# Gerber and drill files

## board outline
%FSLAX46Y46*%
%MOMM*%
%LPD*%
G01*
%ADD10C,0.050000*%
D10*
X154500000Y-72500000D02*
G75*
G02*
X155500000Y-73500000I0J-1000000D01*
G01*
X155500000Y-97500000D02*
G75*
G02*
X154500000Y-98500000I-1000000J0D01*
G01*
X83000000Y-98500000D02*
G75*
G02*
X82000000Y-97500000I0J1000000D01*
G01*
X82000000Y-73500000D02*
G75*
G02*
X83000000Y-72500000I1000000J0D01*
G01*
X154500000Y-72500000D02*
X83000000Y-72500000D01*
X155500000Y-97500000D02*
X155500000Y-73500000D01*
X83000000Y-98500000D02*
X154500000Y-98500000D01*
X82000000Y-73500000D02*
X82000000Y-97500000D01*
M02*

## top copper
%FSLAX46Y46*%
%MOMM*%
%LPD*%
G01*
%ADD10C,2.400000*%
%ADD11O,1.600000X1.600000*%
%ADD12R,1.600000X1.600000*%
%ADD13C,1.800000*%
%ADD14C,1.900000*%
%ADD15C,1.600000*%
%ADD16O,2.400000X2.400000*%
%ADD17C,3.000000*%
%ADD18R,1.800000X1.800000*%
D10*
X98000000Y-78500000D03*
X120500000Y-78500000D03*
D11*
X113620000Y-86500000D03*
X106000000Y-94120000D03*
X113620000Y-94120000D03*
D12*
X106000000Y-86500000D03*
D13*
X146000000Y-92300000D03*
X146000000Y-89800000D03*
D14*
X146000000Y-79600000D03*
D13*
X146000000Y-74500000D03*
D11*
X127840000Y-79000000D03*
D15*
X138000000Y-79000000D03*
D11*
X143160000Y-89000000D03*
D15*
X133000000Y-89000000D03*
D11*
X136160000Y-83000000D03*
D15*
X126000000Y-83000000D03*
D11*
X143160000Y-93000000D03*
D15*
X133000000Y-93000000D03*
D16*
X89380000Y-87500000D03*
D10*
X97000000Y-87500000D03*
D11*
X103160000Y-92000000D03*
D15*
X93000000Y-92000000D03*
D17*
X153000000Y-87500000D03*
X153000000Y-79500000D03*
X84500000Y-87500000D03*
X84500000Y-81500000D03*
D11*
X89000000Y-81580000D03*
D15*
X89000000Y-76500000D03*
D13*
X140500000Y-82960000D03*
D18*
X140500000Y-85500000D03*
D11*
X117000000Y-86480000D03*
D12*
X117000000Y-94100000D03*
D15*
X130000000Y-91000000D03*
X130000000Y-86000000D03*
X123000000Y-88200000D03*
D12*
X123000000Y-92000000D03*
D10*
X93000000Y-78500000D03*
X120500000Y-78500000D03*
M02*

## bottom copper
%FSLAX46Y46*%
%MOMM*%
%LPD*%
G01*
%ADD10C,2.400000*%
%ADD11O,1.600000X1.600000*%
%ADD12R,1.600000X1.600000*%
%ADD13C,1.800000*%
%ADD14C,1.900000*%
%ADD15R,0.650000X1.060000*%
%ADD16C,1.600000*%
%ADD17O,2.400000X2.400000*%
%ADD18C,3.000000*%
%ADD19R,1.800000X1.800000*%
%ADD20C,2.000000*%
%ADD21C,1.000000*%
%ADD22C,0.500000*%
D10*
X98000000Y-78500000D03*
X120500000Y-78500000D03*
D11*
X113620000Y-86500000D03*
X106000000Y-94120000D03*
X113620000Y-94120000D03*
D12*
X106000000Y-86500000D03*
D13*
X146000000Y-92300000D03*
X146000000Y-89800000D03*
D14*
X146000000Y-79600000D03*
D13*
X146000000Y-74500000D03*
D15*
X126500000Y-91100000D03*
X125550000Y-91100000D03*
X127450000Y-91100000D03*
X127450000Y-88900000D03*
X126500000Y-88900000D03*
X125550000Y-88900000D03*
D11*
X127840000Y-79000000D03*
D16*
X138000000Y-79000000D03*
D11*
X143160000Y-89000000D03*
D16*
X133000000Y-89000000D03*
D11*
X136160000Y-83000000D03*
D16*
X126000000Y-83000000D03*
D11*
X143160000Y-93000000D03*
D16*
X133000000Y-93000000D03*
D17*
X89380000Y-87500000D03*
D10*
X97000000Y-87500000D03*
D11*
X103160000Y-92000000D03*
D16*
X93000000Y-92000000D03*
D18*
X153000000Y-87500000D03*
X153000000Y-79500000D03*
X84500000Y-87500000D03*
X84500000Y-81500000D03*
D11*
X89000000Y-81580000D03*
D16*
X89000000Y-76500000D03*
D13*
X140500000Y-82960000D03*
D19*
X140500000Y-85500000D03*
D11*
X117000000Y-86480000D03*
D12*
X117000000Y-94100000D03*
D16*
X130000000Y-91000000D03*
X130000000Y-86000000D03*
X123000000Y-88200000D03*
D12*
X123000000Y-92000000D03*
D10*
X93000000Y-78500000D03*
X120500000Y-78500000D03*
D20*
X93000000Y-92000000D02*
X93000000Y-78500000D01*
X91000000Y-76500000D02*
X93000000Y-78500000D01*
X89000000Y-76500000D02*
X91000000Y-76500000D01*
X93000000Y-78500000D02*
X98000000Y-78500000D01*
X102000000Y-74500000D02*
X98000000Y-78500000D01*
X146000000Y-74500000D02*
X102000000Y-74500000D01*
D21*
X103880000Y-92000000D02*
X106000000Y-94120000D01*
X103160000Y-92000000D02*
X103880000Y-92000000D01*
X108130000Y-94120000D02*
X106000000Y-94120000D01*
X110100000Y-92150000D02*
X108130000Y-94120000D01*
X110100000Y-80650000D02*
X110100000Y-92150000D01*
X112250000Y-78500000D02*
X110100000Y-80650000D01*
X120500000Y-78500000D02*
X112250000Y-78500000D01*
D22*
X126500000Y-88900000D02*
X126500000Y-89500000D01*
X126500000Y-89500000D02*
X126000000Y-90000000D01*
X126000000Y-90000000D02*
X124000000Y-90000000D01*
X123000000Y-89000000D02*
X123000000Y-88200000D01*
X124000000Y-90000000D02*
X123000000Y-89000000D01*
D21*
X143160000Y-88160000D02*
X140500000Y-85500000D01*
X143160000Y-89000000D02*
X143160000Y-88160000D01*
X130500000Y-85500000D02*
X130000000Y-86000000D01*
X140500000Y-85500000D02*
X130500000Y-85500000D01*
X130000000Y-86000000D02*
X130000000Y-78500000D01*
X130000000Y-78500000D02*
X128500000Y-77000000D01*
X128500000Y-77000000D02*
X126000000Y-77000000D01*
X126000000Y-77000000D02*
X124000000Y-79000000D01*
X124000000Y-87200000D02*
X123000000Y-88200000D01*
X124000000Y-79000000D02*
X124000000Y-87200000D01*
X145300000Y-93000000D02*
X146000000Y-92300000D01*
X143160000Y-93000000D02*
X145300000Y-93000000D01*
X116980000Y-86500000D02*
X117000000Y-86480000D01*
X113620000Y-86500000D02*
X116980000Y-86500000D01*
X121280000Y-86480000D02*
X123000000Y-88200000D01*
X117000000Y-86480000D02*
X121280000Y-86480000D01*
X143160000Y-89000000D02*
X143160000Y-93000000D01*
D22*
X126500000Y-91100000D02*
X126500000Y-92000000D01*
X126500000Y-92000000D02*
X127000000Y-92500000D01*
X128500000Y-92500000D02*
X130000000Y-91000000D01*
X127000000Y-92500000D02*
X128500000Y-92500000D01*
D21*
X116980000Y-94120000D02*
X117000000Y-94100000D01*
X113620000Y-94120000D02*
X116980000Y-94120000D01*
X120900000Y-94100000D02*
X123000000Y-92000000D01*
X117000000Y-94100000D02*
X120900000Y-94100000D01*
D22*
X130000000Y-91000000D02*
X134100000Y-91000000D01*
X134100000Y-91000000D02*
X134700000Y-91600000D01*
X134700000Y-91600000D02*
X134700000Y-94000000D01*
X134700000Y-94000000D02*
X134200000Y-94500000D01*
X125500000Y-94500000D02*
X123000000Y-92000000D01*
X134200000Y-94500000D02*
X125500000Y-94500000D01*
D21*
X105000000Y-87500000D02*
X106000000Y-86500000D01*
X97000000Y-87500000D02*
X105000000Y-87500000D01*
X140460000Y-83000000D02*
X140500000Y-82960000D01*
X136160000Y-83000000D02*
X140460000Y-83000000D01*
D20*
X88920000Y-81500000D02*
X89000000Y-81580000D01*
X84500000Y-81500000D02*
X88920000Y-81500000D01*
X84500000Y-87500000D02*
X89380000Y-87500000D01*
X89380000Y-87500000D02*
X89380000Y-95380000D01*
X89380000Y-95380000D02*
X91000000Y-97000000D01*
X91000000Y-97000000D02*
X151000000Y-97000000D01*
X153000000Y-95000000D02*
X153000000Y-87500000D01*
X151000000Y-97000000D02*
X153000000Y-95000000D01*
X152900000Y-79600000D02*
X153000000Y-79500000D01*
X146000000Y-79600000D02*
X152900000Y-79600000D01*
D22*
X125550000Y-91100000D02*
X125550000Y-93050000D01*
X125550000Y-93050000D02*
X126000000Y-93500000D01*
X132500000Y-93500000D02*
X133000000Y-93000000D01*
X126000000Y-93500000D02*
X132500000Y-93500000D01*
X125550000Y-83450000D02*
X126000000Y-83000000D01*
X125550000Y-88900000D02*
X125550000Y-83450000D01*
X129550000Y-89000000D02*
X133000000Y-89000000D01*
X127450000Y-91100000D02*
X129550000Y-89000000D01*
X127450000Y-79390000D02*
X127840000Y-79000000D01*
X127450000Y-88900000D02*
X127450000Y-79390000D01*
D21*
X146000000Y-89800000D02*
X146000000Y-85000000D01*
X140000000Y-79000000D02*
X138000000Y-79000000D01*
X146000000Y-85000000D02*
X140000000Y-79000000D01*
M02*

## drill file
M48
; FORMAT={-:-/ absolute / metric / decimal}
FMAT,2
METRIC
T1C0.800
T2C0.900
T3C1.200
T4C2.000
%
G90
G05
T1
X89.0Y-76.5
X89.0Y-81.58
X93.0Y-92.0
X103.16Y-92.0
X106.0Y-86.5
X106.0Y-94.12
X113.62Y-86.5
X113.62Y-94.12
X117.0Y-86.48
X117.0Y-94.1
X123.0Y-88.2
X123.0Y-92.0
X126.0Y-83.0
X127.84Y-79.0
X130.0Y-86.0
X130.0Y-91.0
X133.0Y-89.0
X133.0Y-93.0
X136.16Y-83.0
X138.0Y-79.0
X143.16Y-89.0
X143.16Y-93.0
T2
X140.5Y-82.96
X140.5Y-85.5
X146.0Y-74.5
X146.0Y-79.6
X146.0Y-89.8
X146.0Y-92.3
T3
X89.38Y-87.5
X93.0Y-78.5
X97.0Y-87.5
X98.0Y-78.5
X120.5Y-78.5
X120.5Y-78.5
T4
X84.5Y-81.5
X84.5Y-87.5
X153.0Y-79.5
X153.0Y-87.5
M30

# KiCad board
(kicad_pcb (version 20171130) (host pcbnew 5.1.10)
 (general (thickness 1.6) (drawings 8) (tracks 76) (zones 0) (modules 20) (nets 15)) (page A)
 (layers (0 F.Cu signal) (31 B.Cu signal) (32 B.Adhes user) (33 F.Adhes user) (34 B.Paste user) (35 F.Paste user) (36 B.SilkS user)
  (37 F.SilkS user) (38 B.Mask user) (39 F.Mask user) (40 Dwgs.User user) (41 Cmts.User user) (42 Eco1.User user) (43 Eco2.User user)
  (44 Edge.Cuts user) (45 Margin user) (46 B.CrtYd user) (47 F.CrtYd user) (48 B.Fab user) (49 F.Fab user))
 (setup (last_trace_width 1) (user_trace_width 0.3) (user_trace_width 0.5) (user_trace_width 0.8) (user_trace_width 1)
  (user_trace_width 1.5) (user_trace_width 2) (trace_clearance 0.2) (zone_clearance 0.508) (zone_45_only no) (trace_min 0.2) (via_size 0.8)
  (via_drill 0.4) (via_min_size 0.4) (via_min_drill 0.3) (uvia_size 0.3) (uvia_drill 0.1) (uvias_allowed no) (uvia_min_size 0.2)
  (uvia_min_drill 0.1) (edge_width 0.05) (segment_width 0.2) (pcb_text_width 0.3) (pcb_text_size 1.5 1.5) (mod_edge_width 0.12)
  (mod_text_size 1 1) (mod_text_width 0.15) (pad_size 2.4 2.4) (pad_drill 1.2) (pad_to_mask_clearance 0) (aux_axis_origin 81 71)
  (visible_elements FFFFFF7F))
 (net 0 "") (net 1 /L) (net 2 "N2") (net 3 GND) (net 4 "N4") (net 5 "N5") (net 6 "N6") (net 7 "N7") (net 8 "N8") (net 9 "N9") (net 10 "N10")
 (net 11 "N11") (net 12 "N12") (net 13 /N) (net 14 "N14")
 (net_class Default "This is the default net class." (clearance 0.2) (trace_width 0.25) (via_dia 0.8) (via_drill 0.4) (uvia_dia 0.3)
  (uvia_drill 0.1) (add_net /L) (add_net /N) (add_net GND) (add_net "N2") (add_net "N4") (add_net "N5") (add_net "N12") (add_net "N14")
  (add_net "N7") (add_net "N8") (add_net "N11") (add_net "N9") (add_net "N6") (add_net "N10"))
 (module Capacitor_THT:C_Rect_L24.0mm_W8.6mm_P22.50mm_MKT (layer F.Cu) (at 120.5 78.5 180)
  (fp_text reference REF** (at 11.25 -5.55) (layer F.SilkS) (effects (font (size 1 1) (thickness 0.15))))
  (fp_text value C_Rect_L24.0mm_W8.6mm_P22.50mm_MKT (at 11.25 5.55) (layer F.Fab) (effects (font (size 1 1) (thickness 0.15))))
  (pad 2 thru_hole circle (at 22.5 0 180) (size 2.4 2.4) (drill 1.2) (layers *.Cu *.Mask) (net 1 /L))
  (pad 1 thru_hole circle (at 0 0 180) (size 2.4 2.4) (drill 1.2) (layers *.Cu *.Mask) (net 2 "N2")))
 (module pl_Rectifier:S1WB (layer F.Cu) (at 106 86.5)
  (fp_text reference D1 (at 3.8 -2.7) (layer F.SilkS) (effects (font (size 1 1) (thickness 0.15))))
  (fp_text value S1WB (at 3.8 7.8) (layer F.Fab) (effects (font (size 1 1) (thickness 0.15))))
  (pad 4 thru_hole oval (at 7.62 0) (size 1.6 1.6) (drill 0.8) (layers *.Cu *.Mask) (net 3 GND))
  (pad 2 thru_hole oval (at 0 7.62) (size 1.6 1.6) (drill 0.8) (layers *.Cu *.Mask) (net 2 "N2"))
  (pad 3 thru_hole oval (at 7.62 7.62) (size 1.6 1.6) (drill 0.8) (layers *.Cu *.Mask) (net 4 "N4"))
  (pad 1 thru_hole rect (at 0 0) (size 1.6 1.6) (drill 0.8) (layers *.Cu *.Mask) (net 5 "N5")))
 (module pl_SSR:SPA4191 (layer F.Cu) (at 146 74.5 270)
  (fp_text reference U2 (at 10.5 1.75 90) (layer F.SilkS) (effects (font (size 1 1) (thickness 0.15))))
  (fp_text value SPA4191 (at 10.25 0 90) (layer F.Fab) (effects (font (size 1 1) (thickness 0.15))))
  (pad 4 thru_hole circle (at 17.8 0 270) (size 1.8 1.8) (drill 0.9) (layers *.Cu *.Mask) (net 3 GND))
  (pad 3 thru_hole circle (at 15.3 0 270) (size 1.8 1.8) (drill 0.9) (layers *.Cu *.Mask) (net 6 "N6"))
  (pad 2 thru_hole circle (at 5.1 0 270) (size 1.9 1.9) (drill 0.9) (layers *.Cu *.Mask) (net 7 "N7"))
  (pad 1 thru_hole circle (at 0 0 270) (size 1.8 1.8) (drill 0.9) (layers *.Cu *.Mask) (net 1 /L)))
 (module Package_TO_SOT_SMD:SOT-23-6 (layer B.Cu) (at 126.5 90 270)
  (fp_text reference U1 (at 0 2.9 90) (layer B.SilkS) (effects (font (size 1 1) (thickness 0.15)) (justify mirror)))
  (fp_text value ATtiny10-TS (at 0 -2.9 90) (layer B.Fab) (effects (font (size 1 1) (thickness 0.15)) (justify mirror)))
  (pad 5 smd rect (at 1.1 0 270) (size 1.06 0.65) (layers B.Cu B.Paste B.Mask) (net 4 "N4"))
  (pad 6 smd rect (at 1.1 0.95 270) (size 1.06 0.65) (layers B.Cu B.Paste B.Mask) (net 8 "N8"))
  (pad 4 smd rect (at 1.1 -0.95 270) (size 1.06 0.65) (layers B.Cu B.Paste B.Mask) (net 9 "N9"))
  (pad 3 smd rect (at -1.1 -0.95 270) (size 1.06 0.65) (layers B.Cu B.Paste B.Mask) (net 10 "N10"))
  (pad 2 smd rect (at -1.1 0 270) (size 1.06 0.65) (layers B.Cu B.Paste B.Mask) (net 3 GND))
  (pad 1 smd rect (at -1.1 0.95 270) (size 1.06 0.65) (layers B.Cu B.Paste B.Mask) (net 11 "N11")))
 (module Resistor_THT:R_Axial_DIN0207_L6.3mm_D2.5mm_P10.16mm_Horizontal (layer F.Cu) (at 138 79 180)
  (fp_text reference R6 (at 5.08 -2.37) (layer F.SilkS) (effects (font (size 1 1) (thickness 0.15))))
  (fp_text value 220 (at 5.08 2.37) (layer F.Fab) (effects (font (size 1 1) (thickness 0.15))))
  (pad 2 thru_hole oval (at 10.16 0 180) (size 1.6 1.6) (drill 0.8) (layers *.Cu *.Mask) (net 10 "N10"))
  (pad 1 thru_hole circle (at 0 0 180) (size 1.6 1.6) (drill 0.8) (layers *.Cu *.Mask) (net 6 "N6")))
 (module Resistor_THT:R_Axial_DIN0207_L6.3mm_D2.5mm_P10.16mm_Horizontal (layer F.Cu) (at 133 89)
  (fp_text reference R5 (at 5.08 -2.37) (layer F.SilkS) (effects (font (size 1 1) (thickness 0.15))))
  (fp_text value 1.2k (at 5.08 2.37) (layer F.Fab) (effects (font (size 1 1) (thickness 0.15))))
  (pad 2 thru_hole oval (at 10.16 0) (size 1.6 1.6) (drill 0.8) (layers *.Cu *.Mask) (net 3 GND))
  (pad 1 thru_hole circle (at 0 0) (size 1.6 1.6) (drill 0.8) (layers *.Cu *.Mask) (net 9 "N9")))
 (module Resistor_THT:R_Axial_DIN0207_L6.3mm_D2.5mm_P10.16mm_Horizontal (layer F.Cu) (at 126 83)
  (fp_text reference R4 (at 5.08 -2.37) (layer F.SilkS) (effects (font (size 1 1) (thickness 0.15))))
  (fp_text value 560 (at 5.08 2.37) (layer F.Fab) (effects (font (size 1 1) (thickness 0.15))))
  (pad 2 thru_hole oval (at 10.16 0) (size 1.6 1.6) (drill 0.8) (layers *.Cu *.Mask) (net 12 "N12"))
  (pad 1 thru_hole circle (at 0 0) (size 1.6 1.6) (drill 0.8) (layers *.Cu *.Mask) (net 11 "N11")))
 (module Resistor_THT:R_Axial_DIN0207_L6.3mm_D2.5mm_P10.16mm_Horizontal (layer F.Cu) (at 133 93)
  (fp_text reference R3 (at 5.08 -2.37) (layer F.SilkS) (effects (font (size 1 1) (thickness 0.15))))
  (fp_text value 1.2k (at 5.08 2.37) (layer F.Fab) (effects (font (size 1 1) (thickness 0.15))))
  (pad 2 thru_hole oval (at 10.16 0) (size 1.6 1.6) (drill 0.8) (layers *.Cu *.Mask) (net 3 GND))
  (pad 1 thru_hole circle (at 0 0) (size 1.6 1.6) (drill 0.8) (layers *.Cu *.Mask) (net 8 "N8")))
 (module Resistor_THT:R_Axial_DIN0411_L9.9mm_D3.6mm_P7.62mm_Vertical (layer F.Cu) (at 97 87.5 180)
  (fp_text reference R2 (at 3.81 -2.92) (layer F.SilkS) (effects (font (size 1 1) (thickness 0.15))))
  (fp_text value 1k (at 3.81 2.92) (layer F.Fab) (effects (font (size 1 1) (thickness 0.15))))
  (pad 2 thru_hole oval (at 7.62 0 180) (size 2.4 2.4) (drill 1.2) (layers *.Cu *.Mask) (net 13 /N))
  (pad 1 thru_hole circle (at 0 0 180) (size 2.4 2.4) (drill 1.2) (layers *.Cu *.Mask) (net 5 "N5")))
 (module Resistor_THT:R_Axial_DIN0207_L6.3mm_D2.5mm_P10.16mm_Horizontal (layer F.Cu) (at 93 92)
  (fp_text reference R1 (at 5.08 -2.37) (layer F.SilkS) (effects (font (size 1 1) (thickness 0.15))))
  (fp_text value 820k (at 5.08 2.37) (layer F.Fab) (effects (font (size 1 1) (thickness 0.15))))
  (pad 2 thru_hole oval (at 10.16 0) (size 1.6 1.6) (drill 0.8) (layers *.Cu *.Mask) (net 2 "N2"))
  (pad 1 thru_hole circle (at 0 0) (size 1.6 1.6) (drill 0.8) (layers *.Cu *.Mask) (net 1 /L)))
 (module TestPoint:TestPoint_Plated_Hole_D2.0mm (layer F.Cu) (at 153 87.5)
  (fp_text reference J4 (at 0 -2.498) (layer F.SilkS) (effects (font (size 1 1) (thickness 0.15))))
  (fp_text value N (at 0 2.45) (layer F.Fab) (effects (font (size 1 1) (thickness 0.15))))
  (pad 1 thru_hole circle (at 0 0) (size 3 3) (drill 2) (layers *.Cu *.Mask) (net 13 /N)))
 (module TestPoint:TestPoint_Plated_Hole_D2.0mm (layer F.Cu) (at 153 79.5)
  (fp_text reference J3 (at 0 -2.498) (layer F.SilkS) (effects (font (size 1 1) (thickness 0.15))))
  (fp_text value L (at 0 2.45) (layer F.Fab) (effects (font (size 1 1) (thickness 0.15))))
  (pad 1 thru_hole circle (at 0 0) (size 3 3) (drill 2) (layers *.Cu *.Mask) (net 7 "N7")))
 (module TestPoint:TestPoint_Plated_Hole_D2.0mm (layer F.Cu) (at 84.5 87.5)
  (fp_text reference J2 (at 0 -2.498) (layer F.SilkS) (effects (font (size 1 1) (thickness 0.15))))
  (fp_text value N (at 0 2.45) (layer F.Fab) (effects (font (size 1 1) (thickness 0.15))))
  (pad 1 thru_hole circle (at 0 0) (size 3 3) (drill 2) (layers *.Cu *.Mask) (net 13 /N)))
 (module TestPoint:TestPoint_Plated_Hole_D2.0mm (layer F.Cu) (at 84.5 81.5)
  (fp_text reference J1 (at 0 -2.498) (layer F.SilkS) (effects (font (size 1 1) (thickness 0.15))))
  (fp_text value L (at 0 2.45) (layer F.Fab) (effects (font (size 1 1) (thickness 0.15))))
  (pad 1 thru_hole circle (at 0 0) (size 3 3) (drill 2) (layers *.Cu *.Mask) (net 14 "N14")))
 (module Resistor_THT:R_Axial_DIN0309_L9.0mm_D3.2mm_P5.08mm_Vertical (layer F.Cu) (at 89 76.5 270)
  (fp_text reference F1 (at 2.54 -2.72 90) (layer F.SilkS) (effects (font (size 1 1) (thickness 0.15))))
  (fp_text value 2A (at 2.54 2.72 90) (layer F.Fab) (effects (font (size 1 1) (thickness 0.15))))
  (pad 2 thru_hole oval (at 5.08 0 270) (size 1.6 1.6) (drill 0.8) (layers *.Cu *.Mask) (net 14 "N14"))
  (pad 1 thru_hole circle (at 0 0 270) (size 1.6 1.6) (drill 0.8) (layers *.Cu *.Mask) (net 1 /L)))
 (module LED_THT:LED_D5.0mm (layer F.Cu) (at 140.5 85.5 90)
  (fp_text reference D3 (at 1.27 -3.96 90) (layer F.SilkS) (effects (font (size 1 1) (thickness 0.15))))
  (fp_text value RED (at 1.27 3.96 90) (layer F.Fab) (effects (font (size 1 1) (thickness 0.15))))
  (pad 2 thru_hole circle (at 2.54 0 90) (size 1.8 1.8) (drill 0.9) (layers *.Cu *.Mask) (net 12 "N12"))
  (pad 1 thru_hole rect (at 0 0 90) (size 1.8 1.8) (drill 0.9) (layers *.Cu *.Mask) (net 3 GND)))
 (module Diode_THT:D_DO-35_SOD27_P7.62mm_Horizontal (layer F.Cu) (at 117 94.1 90)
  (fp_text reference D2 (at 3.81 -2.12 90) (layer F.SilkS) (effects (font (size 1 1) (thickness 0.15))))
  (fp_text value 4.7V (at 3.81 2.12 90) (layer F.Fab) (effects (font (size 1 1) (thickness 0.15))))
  (pad 2 thru_hole oval (at 7.62 0 90) (size 1.6 1.6) (drill 0.8) (layers *.Cu *.Mask) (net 3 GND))
  (pad 1 thru_hole rect (at 0 0 90) (size 1.6 1.6) (drill 0.8) (layers *.Cu *.Mask) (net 4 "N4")))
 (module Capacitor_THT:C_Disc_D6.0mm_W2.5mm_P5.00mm (layer F.Cu) (at 130 86 270)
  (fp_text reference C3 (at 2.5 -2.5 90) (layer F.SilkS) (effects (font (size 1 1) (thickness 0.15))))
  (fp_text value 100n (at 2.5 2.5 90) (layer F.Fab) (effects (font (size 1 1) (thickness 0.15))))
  (pad 2 thru_hole circle (at 5 0 270) (size 1.6 1.6) (drill 0.8) (layers *.Cu *.Mask) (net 4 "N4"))
  (pad 1 thru_hole circle (at 0 0 270) (size 1.6 1.6) (drill 0.8) (layers *.Cu *.Mask) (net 3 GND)))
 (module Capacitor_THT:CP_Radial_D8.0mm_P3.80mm (layer F.Cu) (at 123 92 90)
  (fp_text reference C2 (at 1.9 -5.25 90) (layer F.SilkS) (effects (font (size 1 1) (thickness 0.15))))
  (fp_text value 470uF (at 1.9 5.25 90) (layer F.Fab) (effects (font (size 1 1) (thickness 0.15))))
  (pad 2 thru_hole circle (at 3.8 0 90) (size 1.6 1.6) (drill 0.8) (layers *.Cu *.Mask) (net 3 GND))
  (pad 1 thru_hole rect (at 0 0 90) (size 1.6 1.6) (drill 0.8) (layers *.Cu *.Mask) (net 4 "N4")))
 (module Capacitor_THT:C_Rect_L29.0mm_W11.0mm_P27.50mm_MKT (layer F.Cu) (at 120.5 78.5 180)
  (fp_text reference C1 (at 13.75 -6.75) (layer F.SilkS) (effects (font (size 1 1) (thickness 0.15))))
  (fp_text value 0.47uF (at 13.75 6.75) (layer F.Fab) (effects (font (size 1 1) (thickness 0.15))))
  (pad 2 thru_hole circle (at 27.5 0 180) (size 2.4 2.4) (drill 1.2) (layers *.Cu *.Mask) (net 1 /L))
  (pad 1 thru_hole circle (at 0 0 180) (size 2.4 2.4) (drill 1.2) (layers *.Cu *.Mask) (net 2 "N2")))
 (gr_arc (start 154.5 73.5) (end 155.5 73.5) (angle -90) (layer Edge.Cuts) (width 0.05))
 (gr_arc (start 154.5 97.5) (end 154.5 98.5) (angle -90) (layer Edge.Cuts) (width 0.05))
 (gr_arc (start 83 97.5) (end 82 97.5) (angle -90) (layer Edge.Cuts) (width 0.05))
 (gr_arc (start 83 73.5) (end 83 72.5) (angle -90) (layer Edge.Cuts) (width 0.05))
 (gr_line (start 154.5 72.5) (end 83 72.5) (layer Edge.Cuts) (width 0.05))
 (gr_line (start 155.5 97.5) (end 155.5 73.5) (layer Edge.Cuts) (width 0.05))
 (gr_line (start 83 98.5) (end 154.5 98.5) (layer Edge.Cuts) (width 0.05))
 (gr_line (start 82 73.5) (end 82 97.5) (layer Edge.Cuts) (width 0.05))
 (segment (start 93 92) (end 93 78.5) (width 2) (layer B.Cu) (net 1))
 (segment (start 91 76.5) (end 93 78.5) (width 2) (layer B.Cu) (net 1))
 (segment (start 89 76.5) (end 91 76.5) (width 2) (layer B.Cu) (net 1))
 (segment (start 93 78.5) (end 98 78.5) (width 2) (layer B.Cu) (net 1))
 (segment (start 102 74.5) (end 98 78.5) (width 2) (layer B.Cu) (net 1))
 (segment (start 146 74.5) (end 102 74.5) (width 2) (layer B.Cu) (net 1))
 (segment (start 103.88 92) (end 106 94.12) (width 1) (layer B.Cu) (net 2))
 (segment (start 103.16 92) (end 103.88 92) (width 1) (layer B.Cu) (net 2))
 (segment (start 108.13 94.12) (end 106 94.12) (width 1) (layer B.Cu) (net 2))
 (segment (start 110.1 92.15) (end 108.13 94.12) (width 1) (layer B.Cu) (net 2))
 (segment (start 110.1 80.65) (end 110.1 92.15) (width 1) (layer B.Cu) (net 2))
 (segment (start 112.25 78.5) (end 110.1 80.65) (width 1) (layer B.Cu) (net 2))
 (segment (start 120.5 78.5) (end 112.25 78.5) (width 1) (layer B.Cu) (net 2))
 (segment (start 126.5 88.9) (end 126.5 89.5) (width 0.5) (layer B.Cu) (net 3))
 (segment (start 126.5 89.5) (end 126 90) (width 0.5) (layer B.Cu) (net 3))
 (segment (start 126 90) (end 124 90) (width 0.5) (layer B.Cu) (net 3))
 (segment (start 123 89) (end 123 88.2) (width 0.5) (layer B.Cu) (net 3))
 (segment (start 124 90) (end 123 89) (width 0.5) (layer B.Cu) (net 3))
 (segment (start 143.16 88.16) (end 140.5 85.5) (width 1) (layer B.Cu) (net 3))
 (segment (start 143.16 89) (end 143.16 88.16) (width 1) (layer B.Cu) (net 3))
 (segment (start 130.5 85.5) (end 130 86) (width 1) (layer B.Cu) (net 3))
 (segment (start 140.5 85.5) (end 130.5 85.5) (width 1) (layer B.Cu) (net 3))
 (segment (start 130 86) (end 130 78.5) (width 1) (layer B.Cu) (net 3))
 (segment (start 130 78.5) (end 128.5 77) (width 1) (layer B.Cu) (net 3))
 (segment (start 128.5 77) (end 126 77) (width 1) (layer B.Cu) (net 3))
 (segment (start 126 77) (end 124 79) (width 1) (layer B.Cu) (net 3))
 (segment (start 124 87.2) (end 123 88.2) (width 1) (layer B.Cu) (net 3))
 (segment (start 124 79) (end 124 87.2) (width 1) (layer B.Cu) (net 3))
 (segment (start 145.3 93) (end 146 92.3) (width 1) (layer B.Cu) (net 3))
 (segment (start 143.16 93) (end 145.3 93) (width 1) (layer B.Cu) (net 3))
 (segment (start 116.98 86.5) (end 117 86.48) (width 1) (layer B.Cu) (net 3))
 (segment (start 113.62 86.5) (end 116.98 86.5) (width 1) (layer B.Cu) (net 3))
 (segment (start 121.28 86.48) (end 123 88.2) (width 1) (layer B.Cu) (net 3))
 (segment (start 117 86.48) (end 121.28 86.48) (width 1) (layer B.Cu) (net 3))
 (segment (start 143.16 89) (end 143.16 93) (width 1) (layer B.Cu) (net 3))
 (segment (start 126.5 91.1) (end 126.5 92) (width 0.5) (layer B.Cu) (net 4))
 (segment (start 126.5 92) (end 127 92.5) (width 0.5) (layer B.Cu) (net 4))
 (segment (start 128.5 92.5) (end 130 91) (width 0.5) (layer B.Cu) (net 4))
 (segment (start 127 92.5) (end 128.5 92.5) (width 0.5) (layer B.Cu) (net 4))
 (segment (start 116.98 94.12) (end 117 94.1) (width 1) (layer B.Cu) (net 4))
 (segment (start 113.62 94.12) (end 116.98 94.12) (width 1) (layer B.Cu) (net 4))
 (segment (start 120.9 94.1) (end 123 92) (width 1) (layer B.Cu) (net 4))
 (segment (start 117 94.1) (end 120.9 94.1) (width 1) (layer B.Cu) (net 4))
 (segment (start 130 91) (end 134.1 91) (width 0.5) (layer B.Cu) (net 4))
 (segment (start 134.1 91) (end 134.7 91.6) (width 0.5) (layer B.Cu) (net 4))
 (segment (start 134.7 91.6) (end 134.7 94) (width 0.5) (layer B.Cu) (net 4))
 (segment (start 134.7 94) (end 134.2 94.5) (width 0.5) (layer B.Cu) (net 4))
 (segment (start 125.5 94.5) (end 123 92) (width 0.5) (layer B.Cu) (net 4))
 (segment (start 134.2 94.5) (end 125.5 94.5) (width 0.5) (layer B.Cu) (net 4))
 (segment (start 105 87.5) (end 106 86.5) (width 1) (layer B.Cu) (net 5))
 (segment (start 97 87.5) (end 105 87.5) (width 1) (layer B.Cu) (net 5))
 (segment (start 140.46 83) (end 140.5 82.96) (width 1) (layer B.Cu) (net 12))
 (segment (start 136.16 83) (end 140.46 83) (width 1) (layer B.Cu) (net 12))
 (segment (start 88.92 81.5) (end 89 81.58) (width 2) (layer B.Cu) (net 14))
 (segment (start 84.5 81.5) (end 88.92 81.5) (width 2) (layer B.Cu) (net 14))
 (segment (start 84.5 87.5) (end 89.38 87.5) (width 2) (layer B.Cu) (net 13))
 (segment (start 89.38 87.5) (end 89.38 95.38) (width 2) (layer B.Cu) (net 13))
 (segment (start 89.38 95.38) (end 91 97) (width 2) (layer B.Cu) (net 13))
 (segment (start 91 97) (end 151 97) (width 2) (layer B.Cu) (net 13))
 (segment (start 153 95) (end 153 87.5) (width 2) (layer B.Cu) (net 13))
 (segment (start 151 97) (end 153 95) (width 2) (layer B.Cu) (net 13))
 (segment (start 152.9 79.6) (end 153 79.5) (width 2) (layer B.Cu) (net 7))
 (segment (start 146 79.6) (end 152.9 79.6) (width 2) (layer B.Cu) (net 7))
 (segment (start 125.55 91.1) (end 125.55 93.05) (width 0.5) (layer B.Cu) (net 8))
 (segment (start 125.55 93.05) (end 126 93.5) (width 0.5) (layer B.Cu) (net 8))
 (segment (start 132.5 93.5) (end 133 93) (width 0.5) (layer B.Cu) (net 8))
 (segment (start 126 93.5) (end 132.5 93.5) (width 0.5) (layer B.Cu) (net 8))
 (segment (start 125.55 83.45) (end 126 83) (width 0.5) (layer B.Cu) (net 11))
 (segment (start 125.55 88.9) (end 125.55 83.45) (width 0.5) (layer B.Cu) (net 11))
 (segment (start 129.55 89) (end 133 89) (width 0.5) (layer B.Cu) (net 9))
 (segment (start 127.45 91.1) (end 129.55 89) (width 0.5) (layer B.Cu) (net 9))
 (segment (start 127.45 79.39) (end 127.84 79) (width 0.5) (layer B.Cu) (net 10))
 (segment (start 127.45 88.9) (end 127.45 79.39) (width 0.5) (layer B.Cu) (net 10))
 (segment (start 146 89.8) (end 146 85) (width 1) (layer B.Cu) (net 6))
 (segment (start 140 79) (end 138 79) (width 1) (layer B.Cu) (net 6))
 (segment (start 146 85) (end 140 79) (width 1) (layer B.Cu) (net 6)))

